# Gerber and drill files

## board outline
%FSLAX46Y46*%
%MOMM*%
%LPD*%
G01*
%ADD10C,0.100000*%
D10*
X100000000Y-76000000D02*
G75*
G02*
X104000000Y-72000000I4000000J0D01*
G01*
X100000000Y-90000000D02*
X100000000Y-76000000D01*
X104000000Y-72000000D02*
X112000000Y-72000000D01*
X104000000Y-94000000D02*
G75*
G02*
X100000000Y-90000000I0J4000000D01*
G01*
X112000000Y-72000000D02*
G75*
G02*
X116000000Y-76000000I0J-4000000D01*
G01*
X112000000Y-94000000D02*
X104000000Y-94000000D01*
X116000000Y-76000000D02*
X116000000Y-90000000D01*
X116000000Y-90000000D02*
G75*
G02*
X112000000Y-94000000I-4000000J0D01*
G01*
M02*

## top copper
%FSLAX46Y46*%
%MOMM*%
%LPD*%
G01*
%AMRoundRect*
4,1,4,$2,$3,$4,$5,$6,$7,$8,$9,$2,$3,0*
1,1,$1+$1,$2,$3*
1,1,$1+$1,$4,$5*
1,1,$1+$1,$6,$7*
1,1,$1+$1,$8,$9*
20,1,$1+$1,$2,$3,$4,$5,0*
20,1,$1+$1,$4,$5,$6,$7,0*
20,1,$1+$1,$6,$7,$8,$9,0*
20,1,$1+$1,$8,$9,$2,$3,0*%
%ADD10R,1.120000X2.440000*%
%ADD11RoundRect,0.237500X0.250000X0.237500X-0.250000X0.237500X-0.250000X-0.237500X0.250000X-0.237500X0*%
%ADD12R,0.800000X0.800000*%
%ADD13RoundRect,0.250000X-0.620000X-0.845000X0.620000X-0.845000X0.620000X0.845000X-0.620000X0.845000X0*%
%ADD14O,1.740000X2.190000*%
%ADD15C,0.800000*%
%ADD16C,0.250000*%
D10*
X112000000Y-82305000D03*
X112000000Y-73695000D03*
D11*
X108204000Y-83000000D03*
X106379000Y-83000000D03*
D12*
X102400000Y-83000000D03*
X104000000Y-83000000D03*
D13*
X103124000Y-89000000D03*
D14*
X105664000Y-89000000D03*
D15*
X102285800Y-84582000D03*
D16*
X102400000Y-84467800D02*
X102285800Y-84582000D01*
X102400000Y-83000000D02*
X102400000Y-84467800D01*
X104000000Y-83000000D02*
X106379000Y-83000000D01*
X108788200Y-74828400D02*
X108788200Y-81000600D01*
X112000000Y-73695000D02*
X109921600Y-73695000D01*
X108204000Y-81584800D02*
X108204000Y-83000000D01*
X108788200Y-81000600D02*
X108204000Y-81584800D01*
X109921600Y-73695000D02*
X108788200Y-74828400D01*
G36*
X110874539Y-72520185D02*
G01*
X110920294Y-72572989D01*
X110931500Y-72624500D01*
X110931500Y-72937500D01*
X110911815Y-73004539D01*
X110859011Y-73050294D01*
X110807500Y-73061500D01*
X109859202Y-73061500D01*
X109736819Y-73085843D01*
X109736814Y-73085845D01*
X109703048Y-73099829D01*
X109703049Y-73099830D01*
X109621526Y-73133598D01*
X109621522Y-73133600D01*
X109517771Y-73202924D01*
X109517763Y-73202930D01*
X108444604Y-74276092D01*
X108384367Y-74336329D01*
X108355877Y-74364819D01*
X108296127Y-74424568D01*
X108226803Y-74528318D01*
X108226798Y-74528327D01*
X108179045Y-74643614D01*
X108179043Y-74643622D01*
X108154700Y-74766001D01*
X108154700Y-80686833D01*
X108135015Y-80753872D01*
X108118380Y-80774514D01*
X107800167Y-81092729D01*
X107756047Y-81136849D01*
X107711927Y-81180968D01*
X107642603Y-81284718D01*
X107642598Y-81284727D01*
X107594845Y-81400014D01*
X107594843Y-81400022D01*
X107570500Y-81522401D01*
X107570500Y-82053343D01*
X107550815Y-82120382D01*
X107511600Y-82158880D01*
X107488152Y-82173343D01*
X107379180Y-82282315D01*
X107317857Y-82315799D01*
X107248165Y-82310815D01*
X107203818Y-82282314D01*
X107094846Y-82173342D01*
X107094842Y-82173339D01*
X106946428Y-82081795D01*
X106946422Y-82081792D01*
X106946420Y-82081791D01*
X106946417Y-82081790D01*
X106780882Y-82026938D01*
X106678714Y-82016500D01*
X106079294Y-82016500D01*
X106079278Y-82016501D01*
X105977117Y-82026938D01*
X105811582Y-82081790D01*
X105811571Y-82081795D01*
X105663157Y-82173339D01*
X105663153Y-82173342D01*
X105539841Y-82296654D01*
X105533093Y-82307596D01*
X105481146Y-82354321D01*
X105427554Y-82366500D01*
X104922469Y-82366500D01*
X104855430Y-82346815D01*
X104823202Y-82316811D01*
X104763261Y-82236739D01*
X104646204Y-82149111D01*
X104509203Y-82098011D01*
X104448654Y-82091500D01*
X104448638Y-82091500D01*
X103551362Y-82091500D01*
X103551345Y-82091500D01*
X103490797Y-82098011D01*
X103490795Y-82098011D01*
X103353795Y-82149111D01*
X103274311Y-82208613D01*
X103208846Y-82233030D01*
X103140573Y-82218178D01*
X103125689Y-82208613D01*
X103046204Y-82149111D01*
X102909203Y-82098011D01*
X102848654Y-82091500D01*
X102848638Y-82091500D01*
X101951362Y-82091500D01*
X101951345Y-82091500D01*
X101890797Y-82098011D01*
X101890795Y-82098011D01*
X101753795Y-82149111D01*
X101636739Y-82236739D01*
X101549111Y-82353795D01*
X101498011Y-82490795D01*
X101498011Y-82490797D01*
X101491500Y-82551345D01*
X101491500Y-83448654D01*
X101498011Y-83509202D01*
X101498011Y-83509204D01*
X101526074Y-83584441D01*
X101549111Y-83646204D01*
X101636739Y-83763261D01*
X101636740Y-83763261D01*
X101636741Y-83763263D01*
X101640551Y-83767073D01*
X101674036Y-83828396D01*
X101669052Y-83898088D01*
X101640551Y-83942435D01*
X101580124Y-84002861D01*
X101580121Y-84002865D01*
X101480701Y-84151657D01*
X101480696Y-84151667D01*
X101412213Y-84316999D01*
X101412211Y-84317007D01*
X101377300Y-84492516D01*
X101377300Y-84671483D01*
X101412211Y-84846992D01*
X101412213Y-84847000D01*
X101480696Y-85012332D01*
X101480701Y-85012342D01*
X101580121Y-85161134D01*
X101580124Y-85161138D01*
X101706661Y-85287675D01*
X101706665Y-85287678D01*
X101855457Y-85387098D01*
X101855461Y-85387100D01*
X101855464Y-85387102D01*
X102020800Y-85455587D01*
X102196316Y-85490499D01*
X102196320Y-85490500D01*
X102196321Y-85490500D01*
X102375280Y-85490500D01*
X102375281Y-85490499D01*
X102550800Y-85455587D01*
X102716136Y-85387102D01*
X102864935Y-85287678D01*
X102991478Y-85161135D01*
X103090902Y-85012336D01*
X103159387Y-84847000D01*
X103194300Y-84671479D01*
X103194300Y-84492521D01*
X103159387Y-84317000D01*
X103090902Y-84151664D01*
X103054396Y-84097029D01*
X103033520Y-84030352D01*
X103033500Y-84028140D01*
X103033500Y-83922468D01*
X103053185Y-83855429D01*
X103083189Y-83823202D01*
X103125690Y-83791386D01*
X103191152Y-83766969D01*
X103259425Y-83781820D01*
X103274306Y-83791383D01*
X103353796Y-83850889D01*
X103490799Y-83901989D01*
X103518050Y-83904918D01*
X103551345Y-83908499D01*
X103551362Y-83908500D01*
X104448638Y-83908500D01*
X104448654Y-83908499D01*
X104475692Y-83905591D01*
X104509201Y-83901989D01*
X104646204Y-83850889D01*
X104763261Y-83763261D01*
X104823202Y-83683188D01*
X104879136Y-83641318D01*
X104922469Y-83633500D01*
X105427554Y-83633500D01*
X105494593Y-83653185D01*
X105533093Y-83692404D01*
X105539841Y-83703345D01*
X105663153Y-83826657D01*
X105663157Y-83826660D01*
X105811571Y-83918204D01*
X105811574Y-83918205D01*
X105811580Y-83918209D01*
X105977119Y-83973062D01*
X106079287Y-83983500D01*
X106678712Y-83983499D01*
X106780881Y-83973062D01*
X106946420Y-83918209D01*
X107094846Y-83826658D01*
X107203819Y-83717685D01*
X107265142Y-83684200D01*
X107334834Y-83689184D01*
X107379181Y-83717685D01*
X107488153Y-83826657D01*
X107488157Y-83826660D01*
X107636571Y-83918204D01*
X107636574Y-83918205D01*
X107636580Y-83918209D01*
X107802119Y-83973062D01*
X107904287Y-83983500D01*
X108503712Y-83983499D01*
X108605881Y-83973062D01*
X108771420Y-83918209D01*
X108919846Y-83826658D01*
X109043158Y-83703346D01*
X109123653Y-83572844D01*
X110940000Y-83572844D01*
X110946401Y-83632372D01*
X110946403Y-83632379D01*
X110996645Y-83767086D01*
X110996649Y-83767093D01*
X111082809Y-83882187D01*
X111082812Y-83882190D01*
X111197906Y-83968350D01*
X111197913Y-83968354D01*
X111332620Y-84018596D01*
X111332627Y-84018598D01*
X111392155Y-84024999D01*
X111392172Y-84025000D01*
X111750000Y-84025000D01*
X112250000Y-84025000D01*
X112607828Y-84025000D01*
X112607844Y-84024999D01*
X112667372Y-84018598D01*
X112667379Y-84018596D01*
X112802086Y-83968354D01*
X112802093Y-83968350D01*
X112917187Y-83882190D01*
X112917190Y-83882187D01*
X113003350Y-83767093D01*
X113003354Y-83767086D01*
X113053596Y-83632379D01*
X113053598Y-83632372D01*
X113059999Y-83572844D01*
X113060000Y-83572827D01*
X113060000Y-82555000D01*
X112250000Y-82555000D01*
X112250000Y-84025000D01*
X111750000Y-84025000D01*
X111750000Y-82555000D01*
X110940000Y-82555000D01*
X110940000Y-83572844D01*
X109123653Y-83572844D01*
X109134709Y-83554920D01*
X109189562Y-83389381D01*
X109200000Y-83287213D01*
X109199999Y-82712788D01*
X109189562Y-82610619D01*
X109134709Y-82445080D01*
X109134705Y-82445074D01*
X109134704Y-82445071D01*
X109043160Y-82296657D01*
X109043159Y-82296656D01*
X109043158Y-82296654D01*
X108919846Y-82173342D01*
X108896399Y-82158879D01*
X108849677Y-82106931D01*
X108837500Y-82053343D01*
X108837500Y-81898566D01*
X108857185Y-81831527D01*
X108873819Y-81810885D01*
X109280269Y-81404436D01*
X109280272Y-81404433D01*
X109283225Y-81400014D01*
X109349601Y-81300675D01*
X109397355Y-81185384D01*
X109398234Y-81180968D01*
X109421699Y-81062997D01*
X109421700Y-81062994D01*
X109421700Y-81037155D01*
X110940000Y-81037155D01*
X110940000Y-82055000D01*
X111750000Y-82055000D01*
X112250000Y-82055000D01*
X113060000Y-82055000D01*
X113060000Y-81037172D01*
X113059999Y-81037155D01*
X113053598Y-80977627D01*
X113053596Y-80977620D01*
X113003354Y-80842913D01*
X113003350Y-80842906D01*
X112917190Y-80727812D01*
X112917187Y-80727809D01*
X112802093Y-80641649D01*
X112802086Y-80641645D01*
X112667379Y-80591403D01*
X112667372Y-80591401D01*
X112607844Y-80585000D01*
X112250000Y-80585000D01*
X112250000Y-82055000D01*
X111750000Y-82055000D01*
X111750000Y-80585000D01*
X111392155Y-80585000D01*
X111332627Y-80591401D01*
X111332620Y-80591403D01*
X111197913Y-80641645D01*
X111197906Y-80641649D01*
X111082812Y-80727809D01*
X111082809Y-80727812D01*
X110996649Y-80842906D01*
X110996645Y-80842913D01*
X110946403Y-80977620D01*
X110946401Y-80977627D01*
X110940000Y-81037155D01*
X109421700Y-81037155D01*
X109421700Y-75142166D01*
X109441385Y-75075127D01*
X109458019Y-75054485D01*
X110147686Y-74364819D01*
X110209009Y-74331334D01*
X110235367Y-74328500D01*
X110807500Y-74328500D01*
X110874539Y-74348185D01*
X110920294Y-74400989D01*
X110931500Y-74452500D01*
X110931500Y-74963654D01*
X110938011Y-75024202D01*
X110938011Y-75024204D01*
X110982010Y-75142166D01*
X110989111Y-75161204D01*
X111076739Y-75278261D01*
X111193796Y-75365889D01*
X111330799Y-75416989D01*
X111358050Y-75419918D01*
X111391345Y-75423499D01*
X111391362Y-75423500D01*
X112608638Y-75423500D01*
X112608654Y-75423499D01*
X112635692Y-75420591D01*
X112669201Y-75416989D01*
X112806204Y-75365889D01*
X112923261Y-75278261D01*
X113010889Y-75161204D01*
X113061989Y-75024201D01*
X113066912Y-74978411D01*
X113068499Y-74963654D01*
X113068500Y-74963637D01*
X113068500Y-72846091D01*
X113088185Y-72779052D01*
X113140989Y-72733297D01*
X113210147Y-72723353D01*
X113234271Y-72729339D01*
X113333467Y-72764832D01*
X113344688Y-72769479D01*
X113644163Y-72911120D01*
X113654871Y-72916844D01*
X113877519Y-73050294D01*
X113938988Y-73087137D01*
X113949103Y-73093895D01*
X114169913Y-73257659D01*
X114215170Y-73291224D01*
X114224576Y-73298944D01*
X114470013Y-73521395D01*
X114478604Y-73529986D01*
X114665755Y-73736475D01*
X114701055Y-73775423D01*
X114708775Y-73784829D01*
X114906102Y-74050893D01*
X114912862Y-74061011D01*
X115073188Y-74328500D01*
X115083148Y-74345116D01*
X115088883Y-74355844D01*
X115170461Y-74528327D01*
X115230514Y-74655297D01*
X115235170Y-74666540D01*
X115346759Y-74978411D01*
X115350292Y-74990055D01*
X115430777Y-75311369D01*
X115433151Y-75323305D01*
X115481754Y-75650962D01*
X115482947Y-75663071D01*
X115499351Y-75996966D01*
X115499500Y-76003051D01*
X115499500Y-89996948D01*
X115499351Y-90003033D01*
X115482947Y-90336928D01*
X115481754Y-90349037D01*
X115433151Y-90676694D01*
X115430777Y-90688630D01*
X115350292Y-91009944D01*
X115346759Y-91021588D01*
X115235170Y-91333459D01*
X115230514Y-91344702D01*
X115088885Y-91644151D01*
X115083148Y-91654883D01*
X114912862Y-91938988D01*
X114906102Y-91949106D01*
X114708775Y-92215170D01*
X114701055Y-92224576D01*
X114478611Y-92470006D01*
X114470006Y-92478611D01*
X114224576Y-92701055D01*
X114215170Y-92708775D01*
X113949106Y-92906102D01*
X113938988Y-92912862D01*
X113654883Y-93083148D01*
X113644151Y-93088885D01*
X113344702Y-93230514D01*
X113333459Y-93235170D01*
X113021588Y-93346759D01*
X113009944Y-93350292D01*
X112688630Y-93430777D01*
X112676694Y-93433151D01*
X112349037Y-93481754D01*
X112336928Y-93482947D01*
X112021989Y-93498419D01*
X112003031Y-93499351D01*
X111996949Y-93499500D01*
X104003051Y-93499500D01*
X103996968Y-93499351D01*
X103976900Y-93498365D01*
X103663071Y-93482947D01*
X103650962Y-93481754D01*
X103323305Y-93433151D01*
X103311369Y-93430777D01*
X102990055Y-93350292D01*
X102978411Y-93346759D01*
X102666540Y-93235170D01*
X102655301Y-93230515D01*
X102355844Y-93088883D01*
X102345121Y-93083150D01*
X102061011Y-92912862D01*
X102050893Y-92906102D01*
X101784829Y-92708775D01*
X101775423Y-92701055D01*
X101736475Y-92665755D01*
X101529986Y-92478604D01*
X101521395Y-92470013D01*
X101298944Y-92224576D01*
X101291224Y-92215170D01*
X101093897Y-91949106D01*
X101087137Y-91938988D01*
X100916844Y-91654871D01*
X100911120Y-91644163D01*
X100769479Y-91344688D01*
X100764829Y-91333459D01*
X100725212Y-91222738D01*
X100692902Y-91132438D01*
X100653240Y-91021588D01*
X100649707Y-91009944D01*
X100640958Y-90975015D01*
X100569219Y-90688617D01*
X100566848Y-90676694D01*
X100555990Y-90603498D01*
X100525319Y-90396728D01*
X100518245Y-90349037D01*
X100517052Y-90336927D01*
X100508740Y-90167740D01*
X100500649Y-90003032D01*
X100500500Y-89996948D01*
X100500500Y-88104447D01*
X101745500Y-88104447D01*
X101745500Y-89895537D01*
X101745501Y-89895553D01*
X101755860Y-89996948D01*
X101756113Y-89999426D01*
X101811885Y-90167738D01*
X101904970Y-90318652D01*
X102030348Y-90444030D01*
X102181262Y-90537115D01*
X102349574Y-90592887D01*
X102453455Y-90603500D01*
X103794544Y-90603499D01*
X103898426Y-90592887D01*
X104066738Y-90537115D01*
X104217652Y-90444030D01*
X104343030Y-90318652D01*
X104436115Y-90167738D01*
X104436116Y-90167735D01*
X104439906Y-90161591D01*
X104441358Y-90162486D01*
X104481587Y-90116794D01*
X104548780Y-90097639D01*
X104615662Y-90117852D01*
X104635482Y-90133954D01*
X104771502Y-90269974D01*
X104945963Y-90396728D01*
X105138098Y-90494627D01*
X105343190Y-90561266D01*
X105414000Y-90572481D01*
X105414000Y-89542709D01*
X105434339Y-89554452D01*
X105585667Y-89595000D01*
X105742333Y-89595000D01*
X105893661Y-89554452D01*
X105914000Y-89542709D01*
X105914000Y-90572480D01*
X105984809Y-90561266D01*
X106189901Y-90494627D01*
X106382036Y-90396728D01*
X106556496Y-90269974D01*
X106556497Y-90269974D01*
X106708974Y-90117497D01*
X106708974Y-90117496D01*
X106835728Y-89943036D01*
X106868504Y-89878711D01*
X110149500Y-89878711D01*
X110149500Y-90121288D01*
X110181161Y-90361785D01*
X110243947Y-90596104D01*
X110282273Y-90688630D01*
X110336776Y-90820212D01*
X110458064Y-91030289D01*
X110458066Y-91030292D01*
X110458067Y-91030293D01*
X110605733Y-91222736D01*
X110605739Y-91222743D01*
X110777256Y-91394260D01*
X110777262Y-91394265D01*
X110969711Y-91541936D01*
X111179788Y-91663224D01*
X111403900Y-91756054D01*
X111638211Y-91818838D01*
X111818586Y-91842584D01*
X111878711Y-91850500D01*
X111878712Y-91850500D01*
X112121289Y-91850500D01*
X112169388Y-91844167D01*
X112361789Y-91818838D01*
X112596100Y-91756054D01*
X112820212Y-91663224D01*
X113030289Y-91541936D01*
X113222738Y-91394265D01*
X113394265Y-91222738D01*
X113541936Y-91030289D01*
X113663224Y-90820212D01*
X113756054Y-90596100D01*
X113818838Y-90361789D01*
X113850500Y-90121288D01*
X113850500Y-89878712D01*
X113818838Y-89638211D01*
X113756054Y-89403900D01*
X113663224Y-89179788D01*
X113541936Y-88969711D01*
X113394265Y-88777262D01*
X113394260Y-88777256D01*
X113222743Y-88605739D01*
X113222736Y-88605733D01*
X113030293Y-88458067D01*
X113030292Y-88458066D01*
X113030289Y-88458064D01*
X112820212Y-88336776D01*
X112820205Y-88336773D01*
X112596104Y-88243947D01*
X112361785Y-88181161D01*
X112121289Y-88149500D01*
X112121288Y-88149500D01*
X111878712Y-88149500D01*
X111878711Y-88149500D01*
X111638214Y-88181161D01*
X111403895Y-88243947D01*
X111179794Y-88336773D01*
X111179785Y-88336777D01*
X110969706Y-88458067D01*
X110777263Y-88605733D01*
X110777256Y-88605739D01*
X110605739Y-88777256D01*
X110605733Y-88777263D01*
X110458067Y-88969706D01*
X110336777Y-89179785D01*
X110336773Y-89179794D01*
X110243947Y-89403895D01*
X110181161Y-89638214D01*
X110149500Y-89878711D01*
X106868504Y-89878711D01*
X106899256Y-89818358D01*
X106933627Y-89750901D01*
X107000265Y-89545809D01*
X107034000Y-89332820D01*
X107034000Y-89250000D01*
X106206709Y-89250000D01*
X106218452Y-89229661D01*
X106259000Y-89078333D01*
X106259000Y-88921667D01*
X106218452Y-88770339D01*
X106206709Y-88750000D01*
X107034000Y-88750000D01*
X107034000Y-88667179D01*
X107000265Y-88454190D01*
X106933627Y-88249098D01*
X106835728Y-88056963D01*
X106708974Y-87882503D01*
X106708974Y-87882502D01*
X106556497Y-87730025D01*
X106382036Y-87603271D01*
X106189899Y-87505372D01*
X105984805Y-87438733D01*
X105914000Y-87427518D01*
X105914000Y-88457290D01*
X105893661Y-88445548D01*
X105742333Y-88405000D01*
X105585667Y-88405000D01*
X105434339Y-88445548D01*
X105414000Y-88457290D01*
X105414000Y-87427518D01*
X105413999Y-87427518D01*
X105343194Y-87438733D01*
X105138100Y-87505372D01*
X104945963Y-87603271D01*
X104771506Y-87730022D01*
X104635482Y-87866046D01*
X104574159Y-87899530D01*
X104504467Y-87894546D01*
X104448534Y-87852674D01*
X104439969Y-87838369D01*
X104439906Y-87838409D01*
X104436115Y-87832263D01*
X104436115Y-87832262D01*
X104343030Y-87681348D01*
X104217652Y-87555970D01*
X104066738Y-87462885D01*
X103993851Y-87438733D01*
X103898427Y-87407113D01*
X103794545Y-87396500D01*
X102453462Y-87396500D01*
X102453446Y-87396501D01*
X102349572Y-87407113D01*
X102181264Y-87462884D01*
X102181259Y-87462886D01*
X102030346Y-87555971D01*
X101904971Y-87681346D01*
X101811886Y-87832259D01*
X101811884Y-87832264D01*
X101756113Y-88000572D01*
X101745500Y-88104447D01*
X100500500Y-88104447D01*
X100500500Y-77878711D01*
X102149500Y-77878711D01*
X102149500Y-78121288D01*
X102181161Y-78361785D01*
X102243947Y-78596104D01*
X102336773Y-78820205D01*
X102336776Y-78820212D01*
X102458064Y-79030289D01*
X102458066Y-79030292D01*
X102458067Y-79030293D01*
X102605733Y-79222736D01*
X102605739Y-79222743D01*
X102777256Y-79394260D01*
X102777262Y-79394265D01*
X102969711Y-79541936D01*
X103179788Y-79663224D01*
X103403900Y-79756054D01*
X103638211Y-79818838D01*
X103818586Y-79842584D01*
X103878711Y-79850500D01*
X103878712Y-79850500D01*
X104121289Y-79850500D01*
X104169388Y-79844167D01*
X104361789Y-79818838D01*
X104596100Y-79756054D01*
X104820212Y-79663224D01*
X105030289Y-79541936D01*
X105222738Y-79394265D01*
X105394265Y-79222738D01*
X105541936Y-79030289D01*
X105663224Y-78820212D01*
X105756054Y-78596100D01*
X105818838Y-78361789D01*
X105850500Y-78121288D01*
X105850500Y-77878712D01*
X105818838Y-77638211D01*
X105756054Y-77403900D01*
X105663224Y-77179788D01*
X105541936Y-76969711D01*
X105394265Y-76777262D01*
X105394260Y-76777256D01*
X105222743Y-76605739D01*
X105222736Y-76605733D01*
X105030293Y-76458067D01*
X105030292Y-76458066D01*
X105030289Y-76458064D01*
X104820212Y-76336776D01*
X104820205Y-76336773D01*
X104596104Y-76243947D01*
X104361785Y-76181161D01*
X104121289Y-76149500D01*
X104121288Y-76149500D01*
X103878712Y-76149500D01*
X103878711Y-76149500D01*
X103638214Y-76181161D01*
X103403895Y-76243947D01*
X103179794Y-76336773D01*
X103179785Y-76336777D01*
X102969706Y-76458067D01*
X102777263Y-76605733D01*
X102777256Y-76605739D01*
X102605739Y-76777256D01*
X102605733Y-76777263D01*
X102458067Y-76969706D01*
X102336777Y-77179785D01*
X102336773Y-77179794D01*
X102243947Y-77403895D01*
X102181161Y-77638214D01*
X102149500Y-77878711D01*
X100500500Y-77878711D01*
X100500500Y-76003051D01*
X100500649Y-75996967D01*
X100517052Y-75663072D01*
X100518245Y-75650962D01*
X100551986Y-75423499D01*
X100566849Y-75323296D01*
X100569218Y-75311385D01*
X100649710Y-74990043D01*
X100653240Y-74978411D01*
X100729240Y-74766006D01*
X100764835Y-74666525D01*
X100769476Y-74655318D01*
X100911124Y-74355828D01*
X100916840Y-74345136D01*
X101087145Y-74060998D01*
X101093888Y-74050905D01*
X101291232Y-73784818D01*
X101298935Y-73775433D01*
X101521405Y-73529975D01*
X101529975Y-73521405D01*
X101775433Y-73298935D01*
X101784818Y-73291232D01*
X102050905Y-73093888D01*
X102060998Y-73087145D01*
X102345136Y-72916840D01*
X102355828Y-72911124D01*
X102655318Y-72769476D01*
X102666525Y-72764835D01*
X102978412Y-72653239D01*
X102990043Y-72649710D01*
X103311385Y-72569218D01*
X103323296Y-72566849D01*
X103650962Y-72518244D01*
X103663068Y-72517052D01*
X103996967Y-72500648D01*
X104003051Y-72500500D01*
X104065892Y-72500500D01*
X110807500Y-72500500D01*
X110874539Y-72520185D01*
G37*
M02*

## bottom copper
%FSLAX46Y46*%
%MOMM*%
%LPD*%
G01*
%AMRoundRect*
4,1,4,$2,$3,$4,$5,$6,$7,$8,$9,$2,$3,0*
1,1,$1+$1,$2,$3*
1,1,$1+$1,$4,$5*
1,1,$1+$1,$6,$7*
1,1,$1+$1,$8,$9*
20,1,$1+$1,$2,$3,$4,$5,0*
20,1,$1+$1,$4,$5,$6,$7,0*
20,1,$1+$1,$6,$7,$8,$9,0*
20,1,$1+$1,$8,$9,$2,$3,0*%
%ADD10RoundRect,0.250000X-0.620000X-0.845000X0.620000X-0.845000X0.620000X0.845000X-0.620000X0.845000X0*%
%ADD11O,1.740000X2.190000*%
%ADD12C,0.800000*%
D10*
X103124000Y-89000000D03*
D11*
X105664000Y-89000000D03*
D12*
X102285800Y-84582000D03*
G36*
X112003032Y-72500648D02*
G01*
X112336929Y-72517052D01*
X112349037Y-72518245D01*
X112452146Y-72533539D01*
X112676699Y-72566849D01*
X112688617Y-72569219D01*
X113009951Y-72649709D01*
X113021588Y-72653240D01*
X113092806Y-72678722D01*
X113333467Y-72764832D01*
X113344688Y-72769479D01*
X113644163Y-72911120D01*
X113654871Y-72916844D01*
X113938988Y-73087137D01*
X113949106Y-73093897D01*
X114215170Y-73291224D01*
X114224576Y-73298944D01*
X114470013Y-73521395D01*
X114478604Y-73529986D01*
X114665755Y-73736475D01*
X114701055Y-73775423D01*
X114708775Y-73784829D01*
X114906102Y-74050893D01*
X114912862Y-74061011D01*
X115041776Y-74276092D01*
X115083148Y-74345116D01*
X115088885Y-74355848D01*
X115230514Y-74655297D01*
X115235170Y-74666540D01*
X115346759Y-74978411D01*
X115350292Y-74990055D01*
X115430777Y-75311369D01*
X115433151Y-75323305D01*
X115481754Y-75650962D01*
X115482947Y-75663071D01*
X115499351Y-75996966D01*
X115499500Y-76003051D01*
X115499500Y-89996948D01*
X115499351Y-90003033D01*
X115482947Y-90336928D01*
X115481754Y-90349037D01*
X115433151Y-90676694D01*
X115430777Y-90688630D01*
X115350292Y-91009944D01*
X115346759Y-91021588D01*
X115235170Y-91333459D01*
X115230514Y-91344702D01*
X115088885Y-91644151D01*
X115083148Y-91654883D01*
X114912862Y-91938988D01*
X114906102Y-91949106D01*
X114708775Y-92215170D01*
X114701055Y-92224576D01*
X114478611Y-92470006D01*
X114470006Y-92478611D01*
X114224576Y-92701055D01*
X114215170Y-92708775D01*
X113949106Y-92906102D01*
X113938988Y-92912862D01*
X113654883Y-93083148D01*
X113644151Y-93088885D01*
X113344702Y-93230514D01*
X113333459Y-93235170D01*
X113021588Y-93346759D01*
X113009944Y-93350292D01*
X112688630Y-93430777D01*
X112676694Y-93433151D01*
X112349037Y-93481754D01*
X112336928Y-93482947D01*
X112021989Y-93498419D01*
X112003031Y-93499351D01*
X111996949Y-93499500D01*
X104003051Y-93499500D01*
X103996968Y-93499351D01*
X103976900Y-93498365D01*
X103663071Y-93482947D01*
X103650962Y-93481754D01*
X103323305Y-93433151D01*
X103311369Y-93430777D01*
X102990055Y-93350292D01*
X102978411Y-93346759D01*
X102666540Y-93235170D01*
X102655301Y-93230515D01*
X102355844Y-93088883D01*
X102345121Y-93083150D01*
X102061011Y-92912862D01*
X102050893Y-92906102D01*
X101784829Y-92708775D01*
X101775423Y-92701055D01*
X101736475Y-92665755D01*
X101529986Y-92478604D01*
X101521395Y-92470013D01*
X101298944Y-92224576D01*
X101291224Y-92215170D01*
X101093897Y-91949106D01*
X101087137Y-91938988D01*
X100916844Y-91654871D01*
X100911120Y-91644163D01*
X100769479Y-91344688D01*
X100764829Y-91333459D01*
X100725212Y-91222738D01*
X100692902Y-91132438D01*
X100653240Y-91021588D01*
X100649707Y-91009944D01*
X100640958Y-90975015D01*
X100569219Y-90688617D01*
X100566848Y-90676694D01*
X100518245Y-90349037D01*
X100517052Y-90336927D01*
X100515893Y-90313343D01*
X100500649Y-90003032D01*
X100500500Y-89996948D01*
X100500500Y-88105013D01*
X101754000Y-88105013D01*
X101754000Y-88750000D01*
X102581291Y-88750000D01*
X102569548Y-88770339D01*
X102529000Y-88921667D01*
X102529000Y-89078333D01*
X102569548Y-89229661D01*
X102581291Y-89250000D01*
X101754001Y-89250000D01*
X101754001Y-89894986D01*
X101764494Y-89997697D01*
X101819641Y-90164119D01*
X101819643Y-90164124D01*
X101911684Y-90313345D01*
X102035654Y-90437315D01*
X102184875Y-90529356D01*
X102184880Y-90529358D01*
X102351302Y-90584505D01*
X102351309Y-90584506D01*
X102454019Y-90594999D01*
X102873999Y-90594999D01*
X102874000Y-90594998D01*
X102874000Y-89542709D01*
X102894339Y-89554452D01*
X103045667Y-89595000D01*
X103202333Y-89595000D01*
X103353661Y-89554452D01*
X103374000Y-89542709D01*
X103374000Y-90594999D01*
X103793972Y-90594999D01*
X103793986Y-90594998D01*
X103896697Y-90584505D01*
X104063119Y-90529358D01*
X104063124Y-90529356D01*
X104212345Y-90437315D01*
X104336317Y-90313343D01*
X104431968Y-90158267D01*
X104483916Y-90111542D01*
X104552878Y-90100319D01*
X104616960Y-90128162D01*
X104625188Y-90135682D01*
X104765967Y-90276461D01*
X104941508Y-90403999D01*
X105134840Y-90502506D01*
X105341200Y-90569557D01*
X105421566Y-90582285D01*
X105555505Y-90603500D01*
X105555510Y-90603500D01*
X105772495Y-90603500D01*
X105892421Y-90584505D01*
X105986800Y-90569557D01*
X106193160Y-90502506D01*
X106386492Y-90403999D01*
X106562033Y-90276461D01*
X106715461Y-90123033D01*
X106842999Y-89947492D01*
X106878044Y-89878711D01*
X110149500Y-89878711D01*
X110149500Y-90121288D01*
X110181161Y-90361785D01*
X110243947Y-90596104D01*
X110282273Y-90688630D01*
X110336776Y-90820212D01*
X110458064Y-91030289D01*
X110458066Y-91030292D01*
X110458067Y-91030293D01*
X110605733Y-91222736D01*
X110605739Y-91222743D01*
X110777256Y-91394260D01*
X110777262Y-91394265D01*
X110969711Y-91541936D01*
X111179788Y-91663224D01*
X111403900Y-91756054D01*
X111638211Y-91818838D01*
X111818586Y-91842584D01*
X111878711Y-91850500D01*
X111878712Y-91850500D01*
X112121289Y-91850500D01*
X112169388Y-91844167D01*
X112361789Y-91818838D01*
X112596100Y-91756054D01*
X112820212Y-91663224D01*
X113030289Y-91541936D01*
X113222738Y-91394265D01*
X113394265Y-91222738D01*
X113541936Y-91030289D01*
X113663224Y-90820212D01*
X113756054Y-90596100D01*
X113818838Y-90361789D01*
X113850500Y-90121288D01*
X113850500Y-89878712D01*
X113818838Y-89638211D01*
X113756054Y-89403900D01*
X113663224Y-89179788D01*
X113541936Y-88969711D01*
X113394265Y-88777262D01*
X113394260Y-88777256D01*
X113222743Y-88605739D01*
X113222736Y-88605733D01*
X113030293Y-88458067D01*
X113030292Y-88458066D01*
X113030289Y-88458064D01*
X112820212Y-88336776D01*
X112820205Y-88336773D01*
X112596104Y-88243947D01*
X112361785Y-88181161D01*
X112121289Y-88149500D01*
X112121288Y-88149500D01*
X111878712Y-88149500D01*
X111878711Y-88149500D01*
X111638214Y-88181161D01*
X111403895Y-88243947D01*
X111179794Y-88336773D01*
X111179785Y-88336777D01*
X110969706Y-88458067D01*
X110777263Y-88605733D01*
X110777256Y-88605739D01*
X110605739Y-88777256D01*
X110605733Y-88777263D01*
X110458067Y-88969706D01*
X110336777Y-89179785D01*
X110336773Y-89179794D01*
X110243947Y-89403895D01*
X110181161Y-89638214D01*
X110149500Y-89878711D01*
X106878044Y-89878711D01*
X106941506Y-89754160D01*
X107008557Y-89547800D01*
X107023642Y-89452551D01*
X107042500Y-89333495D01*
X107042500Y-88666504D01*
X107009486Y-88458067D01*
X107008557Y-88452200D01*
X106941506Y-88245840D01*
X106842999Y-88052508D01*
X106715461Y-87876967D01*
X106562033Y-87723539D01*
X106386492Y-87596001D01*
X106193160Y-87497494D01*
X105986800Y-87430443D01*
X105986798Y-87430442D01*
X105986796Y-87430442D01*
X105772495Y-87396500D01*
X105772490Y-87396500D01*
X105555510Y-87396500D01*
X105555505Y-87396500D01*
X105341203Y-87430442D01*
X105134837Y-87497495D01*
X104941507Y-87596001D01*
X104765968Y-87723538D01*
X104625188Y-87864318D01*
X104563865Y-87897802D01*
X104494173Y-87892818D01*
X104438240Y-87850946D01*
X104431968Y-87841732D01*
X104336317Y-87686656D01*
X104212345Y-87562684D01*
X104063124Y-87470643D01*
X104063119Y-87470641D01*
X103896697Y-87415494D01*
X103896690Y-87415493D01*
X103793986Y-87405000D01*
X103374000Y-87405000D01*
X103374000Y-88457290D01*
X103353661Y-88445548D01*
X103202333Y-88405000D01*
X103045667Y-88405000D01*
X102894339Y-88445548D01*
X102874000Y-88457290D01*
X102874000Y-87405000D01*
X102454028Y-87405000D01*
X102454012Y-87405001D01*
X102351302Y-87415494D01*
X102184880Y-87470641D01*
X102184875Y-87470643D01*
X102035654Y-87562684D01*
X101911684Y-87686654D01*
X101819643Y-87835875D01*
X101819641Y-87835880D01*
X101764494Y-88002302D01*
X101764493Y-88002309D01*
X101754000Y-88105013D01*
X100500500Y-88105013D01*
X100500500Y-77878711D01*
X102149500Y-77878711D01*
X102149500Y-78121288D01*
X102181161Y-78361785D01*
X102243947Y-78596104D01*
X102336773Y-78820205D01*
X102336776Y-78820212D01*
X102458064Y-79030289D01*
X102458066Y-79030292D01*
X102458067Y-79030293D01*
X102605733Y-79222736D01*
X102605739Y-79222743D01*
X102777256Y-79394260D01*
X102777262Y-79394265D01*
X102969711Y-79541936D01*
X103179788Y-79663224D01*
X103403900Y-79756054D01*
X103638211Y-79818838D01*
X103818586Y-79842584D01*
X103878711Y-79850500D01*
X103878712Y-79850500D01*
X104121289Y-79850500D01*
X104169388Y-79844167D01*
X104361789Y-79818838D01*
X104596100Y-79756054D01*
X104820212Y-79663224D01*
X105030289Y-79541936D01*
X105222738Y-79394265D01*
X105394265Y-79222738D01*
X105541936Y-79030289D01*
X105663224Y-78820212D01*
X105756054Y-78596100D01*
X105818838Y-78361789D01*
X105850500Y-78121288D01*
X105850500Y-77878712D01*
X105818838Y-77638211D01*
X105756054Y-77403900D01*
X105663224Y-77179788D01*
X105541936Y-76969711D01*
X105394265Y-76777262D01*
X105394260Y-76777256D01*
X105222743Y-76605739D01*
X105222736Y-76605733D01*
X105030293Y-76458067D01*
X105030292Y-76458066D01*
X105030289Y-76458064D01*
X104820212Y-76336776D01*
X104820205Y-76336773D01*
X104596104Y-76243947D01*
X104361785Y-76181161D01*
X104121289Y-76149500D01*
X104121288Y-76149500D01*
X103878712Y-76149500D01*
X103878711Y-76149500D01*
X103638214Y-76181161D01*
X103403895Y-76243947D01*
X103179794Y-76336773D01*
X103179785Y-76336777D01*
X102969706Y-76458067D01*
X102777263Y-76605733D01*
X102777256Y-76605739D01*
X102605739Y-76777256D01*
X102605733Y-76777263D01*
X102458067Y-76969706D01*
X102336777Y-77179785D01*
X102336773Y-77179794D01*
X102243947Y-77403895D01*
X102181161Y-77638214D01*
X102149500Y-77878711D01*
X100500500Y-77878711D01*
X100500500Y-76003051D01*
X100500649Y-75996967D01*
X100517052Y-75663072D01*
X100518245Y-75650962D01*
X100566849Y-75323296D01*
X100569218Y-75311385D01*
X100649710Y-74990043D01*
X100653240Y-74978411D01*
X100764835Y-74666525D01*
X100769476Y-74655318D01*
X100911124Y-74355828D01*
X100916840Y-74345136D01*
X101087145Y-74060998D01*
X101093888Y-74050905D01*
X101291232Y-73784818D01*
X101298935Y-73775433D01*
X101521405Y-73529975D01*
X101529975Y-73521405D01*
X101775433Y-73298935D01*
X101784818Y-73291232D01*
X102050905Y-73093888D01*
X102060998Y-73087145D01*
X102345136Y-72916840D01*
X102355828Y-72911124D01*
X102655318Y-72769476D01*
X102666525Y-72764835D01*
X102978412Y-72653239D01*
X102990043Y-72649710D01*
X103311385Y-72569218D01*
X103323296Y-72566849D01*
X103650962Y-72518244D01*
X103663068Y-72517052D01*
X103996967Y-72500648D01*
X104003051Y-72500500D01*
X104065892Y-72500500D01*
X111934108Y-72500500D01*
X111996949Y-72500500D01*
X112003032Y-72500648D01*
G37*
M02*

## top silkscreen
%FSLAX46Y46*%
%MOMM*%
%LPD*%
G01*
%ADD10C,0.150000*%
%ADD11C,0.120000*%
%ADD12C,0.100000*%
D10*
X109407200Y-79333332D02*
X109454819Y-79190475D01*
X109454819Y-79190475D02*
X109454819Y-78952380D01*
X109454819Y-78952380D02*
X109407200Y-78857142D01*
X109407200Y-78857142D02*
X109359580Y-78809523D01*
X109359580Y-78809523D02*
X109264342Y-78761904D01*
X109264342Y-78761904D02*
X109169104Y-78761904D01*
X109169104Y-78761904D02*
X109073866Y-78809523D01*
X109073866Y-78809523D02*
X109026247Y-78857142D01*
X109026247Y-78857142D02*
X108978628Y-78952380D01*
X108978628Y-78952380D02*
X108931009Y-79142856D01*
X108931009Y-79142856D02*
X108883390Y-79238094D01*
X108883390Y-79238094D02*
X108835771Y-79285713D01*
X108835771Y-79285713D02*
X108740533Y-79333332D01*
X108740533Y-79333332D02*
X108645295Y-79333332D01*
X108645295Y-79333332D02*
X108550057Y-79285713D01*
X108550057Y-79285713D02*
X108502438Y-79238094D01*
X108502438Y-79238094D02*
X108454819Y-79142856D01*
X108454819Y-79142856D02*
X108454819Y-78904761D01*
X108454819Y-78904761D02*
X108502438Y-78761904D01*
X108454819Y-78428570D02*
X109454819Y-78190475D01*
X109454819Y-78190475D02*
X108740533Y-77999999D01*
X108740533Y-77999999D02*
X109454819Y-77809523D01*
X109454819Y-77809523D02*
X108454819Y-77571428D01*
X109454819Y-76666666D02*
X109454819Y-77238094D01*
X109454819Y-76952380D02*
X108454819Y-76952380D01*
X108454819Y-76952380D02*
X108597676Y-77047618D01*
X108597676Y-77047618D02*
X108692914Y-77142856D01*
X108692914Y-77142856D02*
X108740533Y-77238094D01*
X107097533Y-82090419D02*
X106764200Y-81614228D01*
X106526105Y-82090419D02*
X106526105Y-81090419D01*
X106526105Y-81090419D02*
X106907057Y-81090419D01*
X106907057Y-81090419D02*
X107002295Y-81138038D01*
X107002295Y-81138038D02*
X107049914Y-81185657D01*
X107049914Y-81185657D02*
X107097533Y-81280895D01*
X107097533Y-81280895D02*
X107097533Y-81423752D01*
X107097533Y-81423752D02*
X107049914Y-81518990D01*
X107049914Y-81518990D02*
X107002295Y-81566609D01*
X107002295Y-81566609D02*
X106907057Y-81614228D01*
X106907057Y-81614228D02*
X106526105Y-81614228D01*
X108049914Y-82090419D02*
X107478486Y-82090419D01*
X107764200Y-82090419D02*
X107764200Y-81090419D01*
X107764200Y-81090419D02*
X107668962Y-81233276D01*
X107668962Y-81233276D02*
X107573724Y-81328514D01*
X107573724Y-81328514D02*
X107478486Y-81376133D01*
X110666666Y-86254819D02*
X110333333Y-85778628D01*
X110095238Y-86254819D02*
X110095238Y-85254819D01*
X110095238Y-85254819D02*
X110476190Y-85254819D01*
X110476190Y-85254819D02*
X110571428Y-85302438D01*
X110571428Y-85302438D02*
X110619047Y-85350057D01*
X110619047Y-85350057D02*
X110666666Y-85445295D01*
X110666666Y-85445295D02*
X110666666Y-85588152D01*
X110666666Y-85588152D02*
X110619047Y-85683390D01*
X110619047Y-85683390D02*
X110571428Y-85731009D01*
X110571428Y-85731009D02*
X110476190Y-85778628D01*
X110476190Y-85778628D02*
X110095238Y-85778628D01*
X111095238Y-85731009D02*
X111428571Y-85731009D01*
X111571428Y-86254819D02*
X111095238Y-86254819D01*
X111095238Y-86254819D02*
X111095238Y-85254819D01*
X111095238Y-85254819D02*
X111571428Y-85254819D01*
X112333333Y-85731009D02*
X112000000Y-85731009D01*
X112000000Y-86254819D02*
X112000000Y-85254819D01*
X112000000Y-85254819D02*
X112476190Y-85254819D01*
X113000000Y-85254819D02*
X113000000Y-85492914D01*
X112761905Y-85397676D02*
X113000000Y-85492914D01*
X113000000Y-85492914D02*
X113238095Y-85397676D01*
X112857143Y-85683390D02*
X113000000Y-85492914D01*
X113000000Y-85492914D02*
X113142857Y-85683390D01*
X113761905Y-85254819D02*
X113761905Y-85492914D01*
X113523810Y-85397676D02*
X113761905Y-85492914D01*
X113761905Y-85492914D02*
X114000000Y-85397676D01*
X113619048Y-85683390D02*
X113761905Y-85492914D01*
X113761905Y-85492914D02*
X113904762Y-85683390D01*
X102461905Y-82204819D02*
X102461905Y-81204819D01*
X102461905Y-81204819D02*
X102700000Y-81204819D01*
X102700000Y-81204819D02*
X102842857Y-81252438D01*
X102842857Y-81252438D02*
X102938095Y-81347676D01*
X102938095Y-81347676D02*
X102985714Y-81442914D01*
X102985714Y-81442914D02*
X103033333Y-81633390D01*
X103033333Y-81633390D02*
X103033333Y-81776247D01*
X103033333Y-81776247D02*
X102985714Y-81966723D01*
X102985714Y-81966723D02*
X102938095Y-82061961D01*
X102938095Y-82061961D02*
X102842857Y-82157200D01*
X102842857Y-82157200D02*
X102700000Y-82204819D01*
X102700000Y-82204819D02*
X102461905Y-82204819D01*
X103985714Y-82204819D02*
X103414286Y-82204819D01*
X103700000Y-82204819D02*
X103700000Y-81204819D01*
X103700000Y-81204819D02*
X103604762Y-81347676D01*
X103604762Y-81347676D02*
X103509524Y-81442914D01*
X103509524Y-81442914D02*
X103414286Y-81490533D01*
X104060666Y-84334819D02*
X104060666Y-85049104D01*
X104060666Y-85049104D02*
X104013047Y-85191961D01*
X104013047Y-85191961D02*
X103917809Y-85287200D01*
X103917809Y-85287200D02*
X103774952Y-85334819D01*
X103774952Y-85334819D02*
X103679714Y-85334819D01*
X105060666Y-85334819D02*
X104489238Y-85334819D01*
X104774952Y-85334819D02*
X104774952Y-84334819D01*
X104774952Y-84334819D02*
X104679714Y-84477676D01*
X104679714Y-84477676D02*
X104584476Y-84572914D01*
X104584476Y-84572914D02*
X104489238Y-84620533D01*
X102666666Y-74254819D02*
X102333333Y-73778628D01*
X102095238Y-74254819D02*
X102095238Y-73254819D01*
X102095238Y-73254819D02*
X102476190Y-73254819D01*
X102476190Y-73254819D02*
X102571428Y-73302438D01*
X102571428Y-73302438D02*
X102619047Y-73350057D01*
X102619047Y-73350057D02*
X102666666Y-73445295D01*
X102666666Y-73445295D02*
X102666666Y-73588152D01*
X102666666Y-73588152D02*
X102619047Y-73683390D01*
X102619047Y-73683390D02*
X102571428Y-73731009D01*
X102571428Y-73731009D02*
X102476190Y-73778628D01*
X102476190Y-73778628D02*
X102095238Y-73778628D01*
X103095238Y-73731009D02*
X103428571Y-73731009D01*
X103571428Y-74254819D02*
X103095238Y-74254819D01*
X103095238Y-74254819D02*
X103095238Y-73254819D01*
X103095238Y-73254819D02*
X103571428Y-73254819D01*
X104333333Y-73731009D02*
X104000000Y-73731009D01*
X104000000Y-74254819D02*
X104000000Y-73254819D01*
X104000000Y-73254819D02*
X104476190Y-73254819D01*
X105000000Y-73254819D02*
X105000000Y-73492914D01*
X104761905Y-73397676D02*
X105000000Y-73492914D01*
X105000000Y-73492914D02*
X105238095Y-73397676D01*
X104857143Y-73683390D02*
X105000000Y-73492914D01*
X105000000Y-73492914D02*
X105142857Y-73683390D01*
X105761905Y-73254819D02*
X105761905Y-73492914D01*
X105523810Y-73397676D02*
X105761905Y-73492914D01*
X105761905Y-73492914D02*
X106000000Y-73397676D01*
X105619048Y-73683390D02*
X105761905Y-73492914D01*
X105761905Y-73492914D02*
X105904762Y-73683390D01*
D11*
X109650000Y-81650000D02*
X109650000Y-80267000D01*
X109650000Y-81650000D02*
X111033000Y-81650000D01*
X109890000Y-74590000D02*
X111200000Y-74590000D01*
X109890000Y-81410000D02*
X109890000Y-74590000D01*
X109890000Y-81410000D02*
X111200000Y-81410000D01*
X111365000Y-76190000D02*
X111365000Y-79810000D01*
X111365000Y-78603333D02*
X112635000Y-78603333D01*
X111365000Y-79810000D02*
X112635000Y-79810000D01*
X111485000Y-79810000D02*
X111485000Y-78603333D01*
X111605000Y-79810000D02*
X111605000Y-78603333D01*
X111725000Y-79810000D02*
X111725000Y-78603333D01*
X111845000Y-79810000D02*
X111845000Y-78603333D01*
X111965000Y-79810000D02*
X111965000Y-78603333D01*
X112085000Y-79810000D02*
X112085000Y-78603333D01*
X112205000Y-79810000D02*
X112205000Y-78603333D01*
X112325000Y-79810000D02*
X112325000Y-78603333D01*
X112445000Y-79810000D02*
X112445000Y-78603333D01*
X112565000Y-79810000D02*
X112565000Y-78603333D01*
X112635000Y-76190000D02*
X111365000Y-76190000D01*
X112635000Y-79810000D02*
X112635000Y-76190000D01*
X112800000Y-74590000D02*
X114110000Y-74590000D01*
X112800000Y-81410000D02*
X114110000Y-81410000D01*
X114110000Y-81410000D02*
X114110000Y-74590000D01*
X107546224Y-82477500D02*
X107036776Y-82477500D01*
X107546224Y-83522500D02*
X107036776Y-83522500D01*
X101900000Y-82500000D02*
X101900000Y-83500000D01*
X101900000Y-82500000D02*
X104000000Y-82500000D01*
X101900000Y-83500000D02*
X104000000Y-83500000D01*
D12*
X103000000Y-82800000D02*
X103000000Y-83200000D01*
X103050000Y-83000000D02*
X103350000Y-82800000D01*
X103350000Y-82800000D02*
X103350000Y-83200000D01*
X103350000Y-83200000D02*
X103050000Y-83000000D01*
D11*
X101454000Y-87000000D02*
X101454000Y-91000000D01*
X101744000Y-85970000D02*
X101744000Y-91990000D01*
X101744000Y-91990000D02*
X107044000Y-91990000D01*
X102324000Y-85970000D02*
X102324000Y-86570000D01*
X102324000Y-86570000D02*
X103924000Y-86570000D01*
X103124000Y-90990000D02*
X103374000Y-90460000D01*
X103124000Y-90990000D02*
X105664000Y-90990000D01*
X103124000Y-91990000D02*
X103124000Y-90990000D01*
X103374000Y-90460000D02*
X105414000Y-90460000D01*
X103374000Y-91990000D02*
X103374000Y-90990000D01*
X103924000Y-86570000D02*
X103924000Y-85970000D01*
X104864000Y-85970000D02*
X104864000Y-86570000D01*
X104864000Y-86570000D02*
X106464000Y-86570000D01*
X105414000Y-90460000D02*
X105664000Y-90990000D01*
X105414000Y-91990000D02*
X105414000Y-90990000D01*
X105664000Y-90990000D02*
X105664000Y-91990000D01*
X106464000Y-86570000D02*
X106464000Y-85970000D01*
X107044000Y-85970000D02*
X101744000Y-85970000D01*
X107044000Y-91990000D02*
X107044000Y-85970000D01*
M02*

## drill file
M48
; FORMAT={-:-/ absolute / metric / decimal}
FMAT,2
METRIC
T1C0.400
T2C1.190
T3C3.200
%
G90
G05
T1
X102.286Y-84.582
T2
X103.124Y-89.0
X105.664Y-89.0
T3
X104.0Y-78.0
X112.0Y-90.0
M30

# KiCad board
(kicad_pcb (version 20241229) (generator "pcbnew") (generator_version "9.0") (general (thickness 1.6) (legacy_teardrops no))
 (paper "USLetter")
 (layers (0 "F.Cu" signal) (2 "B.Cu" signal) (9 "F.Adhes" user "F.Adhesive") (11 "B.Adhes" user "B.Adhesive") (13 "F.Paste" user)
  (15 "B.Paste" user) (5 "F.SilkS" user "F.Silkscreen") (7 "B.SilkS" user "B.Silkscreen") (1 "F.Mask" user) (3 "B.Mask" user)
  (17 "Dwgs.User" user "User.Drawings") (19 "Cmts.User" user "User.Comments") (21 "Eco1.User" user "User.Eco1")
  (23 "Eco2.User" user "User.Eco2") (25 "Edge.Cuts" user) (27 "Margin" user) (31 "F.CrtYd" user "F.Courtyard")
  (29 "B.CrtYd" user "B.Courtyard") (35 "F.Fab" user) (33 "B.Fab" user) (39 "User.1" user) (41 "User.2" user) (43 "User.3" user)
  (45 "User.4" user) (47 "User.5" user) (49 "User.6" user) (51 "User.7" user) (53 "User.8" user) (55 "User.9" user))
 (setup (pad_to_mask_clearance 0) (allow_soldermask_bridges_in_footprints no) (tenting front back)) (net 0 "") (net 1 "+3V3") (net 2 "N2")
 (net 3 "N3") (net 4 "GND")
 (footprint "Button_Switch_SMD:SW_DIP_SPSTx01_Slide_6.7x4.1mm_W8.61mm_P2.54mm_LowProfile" (layer "F.Cu") (at 112 78 90)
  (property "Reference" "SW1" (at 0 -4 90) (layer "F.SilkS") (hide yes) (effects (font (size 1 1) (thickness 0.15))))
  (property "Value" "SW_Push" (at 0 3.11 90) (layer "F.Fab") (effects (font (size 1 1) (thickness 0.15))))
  (fp_line (start -3.65 -2.35) (end -2.267 -2.35) (stroke (width 0.12) (type solid)) (layer "F.SilkS"))
  (fp_line (start -3.65 -2.35) (end -3.65 -0.967) (stroke (width 0.12) (type solid)) (layer "F.SilkS"))
  (fp_line (start 3.41 -2.11) (end 3.41 -0.8) (stroke (width 0.12) (type solid)) (layer "F.SilkS"))
  (fp_line (start -3.41 -2.11) (end 3.41 -2.11) (stroke (width 0.12) (type solid)) (layer "F.SilkS"))
  (fp_line (start -3.41 -2.11) (end -3.41 -0.8) (stroke (width 0.12) (type solid)) (layer "F.SilkS"))
  (fp_line (start 1.81 -0.635) (end -1.81 -0.635) (stroke (width 0.12) (type solid)) (layer "F.SilkS"))
  (fp_line (start -0.603333 -0.635) (end -0.603333 0.635) (stroke (width 0.12) (type solid)) (layer "F.SilkS"))
  (fp_line (start -1.81 -0.635) (end -1.81 0.635) (stroke (width 0.12) (type solid)) (layer "F.SilkS"))
  (fp_line (start -1.81 -0.515) (end -0.603333 -0.515) (stroke (width 0.12) (type solid)) (layer "F.SilkS"))
  (fp_line (start -1.81 -0.395) (end -0.603333 -0.395) (stroke (width 0.12) (type solid)) (layer "F.SilkS"))
  (fp_line (start -1.81 -0.275) (end -0.603333 -0.275) (stroke (width 0.12) (type solid)) (layer "F.SilkS"))
  (fp_line (start -1.81 -0.155) (end -0.603333 -0.155) (stroke (width 0.12) (type solid)) (layer "F.SilkS"))
  (fp_line (start -1.81 -0.035) (end -0.603333 -0.035) (stroke (width 0.12) (type solid)) (layer "F.SilkS"))
  (fp_line (start -1.81 0.085) (end -0.603333 0.085) (stroke (width 0.12) (type solid)) (layer "F.SilkS"))
  (fp_line (start -1.81 0.205) (end -0.603333 0.205) (stroke (width 0.12) (type solid)) (layer "F.SilkS"))
  (fp_line (start -1.81 0.325) (end -0.603333 0.325) (stroke (width 0.12) (type solid)) (layer "F.SilkS"))
  (fp_line (start -1.81 0.445) (end -0.603333 0.445) (stroke (width 0.12) (type solid)) (layer "F.SilkS"))
  (fp_line (start -1.81 0.565) (end -0.603333 0.565) (stroke (width 0.12) (type solid)) (layer "F.SilkS"))
  (fp_line (start 1.81 0.635) (end 1.81 -0.635) (stroke (width 0.12) (type solid)) (layer "F.SilkS"))
  (fp_line (start -1.81 0.635) (end 1.81 0.635) (stroke (width 0.12) (type solid)) (layer "F.SilkS"))
  (fp_line (start 3.41 0.8) (end 3.41 2.11) (stroke (width 0.12) (type solid)) (layer "F.SilkS"))
  (fp_line (start -3.41 0.8) (end -3.41 2.11) (stroke (width 0.12) (type solid)) (layer "F.SilkS"))
  (fp_line (start -3.41 2.11) (end 3.41 2.11) (stroke (width 0.12) (type solid)) (layer "F.SilkS"))
  (pad "1" smd rect (at -4.305 0 90) (size 2.44 1.12) (layers "F.Cu" "F.Mask" "F.Paste") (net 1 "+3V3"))
  (pad "2" smd rect (at 4.305 0 90) (size 2.44 1.12) (layers "F.Cu" "F.Mask" "F.Paste") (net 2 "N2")))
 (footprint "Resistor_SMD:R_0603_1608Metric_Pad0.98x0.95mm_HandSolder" (layer "F.Cu") (at 107.2915 83 180)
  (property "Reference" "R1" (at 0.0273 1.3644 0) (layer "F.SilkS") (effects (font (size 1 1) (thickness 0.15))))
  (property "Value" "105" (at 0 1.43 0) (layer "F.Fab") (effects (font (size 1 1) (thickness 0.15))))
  (fp_line (start -0.254724 0.5225) (end 0.254724 0.5225) (stroke (width 0.12) (type solid)) (layer "F.SilkS"))
  (fp_line (start -0.254724 -0.5225) (end 0.254724 -0.5225) (stroke (width 0.12) (type solid)) (layer "F.SilkS"))
  (pad "1" smd roundrect (at -0.9125 0 180) (size 0.975 0.95) (layers "F.Cu" "F.Mask" "F.Paste") (roundrect_rratio 0.25) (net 2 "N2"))
  (pad "2" smd roundrect (at 0.9125 0 180) (size 0.975 0.95) (layers "F.Cu" "F.Mask" "F.Paste") (roundrect_rratio 0.25) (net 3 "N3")))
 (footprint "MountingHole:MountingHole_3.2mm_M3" (layer "F.Cu") (at 112 90)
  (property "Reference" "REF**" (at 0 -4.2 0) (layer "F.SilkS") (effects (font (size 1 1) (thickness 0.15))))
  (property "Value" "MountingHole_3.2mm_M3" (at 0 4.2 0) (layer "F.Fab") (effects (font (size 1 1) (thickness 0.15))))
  (pad "" np_thru_hole circle (at 0 0) (size 3.2 3.2) (drill 3.2) (layers "*.Cu" "*.Mask")))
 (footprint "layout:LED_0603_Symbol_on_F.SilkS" (layer "F.Cu") (at 103.2 83)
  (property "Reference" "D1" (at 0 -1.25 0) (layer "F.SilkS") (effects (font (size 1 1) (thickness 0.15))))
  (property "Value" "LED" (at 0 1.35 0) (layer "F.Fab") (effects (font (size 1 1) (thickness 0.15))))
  (fp_line (start -1.3 -0.5) (end -1.3 0.5) (stroke (width 0.12) (type solid)) (layer "F.SilkS"))
  (fp_line (start -1.3 -0.5) (end 0.8 -0.5) (stroke (width 0.12) (type solid)) (layer "F.SilkS"))
  (fp_line (start -1.3 0.5) (end 0.8 0.5) (stroke (width 0.12) (type solid)) (layer "F.SilkS"))
  (fp_line (start -0.2 -0.2) (end -0.2 0.2) (stroke (width 0.1) (type solid)) (layer "F.SilkS"))
  (fp_line (start -0.15 0) (end 0.15 -0.2) (stroke (width 0.1) (type solid)) (layer "F.SilkS"))
  (fp_line (start 0.15 -0.2) (end 0.15 0.2) (stroke (width 0.1) (type solid)) (layer "F.SilkS"))
  (fp_line (start 0.15 0.2) (end -0.15 0) (stroke (width 0.1) (type solid)) (layer "F.SilkS"))
  (pad "1" smd rect (at -0.8 0 180) (size 0.8 0.8) (layers "F.Cu" "F.Mask" "F.Paste") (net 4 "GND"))
  (pad "2" smd rect (at 0.8 0 180) (size 0.8 0.8) (layers "F.Cu" "F.Mask" "F.Paste") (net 3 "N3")))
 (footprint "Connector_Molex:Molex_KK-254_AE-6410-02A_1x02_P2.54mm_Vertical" (layer "F.Cu") (at 103.124 89)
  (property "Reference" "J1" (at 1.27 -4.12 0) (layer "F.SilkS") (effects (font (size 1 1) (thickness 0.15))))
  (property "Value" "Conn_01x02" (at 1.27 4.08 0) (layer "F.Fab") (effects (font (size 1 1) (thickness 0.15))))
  (fp_line (start -1.67 -2) (end -1.67 2) (stroke (width 0.12) (type solid)) (layer "F.SilkS"))
  (fp_line (start -1.38 -3.03) (end -1.38 2.99) (stroke (width 0.12) (type solid)) (layer "F.SilkS"))
  (fp_line (start -1.38 2.99) (end 3.92 2.99) (stroke (width 0.12) (type solid)) (layer "F.SilkS"))
  (fp_line (start -0.8 -3.03) (end -0.8 -2.43) (stroke (width 0.12) (type solid)) (layer "F.SilkS"))
  (fp_line (start -0.8 -2.43) (end 0.8 -2.43) (stroke (width 0.12) (type solid)) (layer "F.SilkS"))
  (fp_line (start 0 1.99) (end 0.25 1.46) (stroke (width 0.12) (type solid)) (layer "F.SilkS"))
  (fp_line (start 0 1.99) (end 2.54 1.99) (stroke (width 0.12) (type solid)) (layer "F.SilkS"))
  (fp_line (start 0 2.99) (end 0 1.99) (stroke (width 0.12) (type solid)) (layer "F.SilkS"))
  (fp_line (start 0.25 1.46) (end 2.29 1.46) (stroke (width 0.12) (type solid)) (layer "F.SilkS"))
  (fp_line (start 0.25 2.99) (end 0.25 1.99) (stroke (width 0.12) (type solid)) (layer "F.SilkS"))
  (fp_line (start 0.8 -2.43) (end 0.8 -3.03) (stroke (width 0.12) (type solid)) (layer "F.SilkS"))
  (fp_line (start 1.74 -3.03) (end 1.74 -2.43) (stroke (width 0.12) (type solid)) (layer "F.SilkS"))
  (fp_line (start 1.74 -2.43) (end 3.34 -2.43) (stroke (width 0.12) (type solid)) (layer "F.SilkS"))
  (fp_line (start 2.29 1.46) (end 2.54 1.99) (stroke (width 0.12) (type solid)) (layer "F.SilkS"))
  (fp_line (start 2.29 2.99) (end 2.29 1.99) (stroke (width 0.12) (type solid)) (layer "F.SilkS"))
  (fp_line (start 2.54 1.99) (end 2.54 2.99) (stroke (width 0.12) (type solid)) (layer "F.SilkS"))
  (fp_line (start 3.34 -2.43) (end 3.34 -3.03) (stroke (width 0.12) (type solid)) (layer "F.SilkS"))
  (fp_line (start 3.92 -3.03) (end -1.38 -3.03) (stroke (width 0.12) (type solid)) (layer "F.SilkS"))
  (fp_line (start 3.92 2.99) (end 3.92 -3.03) (stroke (width 0.12) (type solid)) (layer "F.SilkS"))
  (pad "1" thru_hole roundrect (at 0 0) (size 1.74 2.19) (drill 1.19) (layers "*.Cu" "*.Mask") (remove_unused_layers no)
   (roundrect_rratio 0.143678) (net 4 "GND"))
  (pad "2" thru_hole oval (at 2.54 0) (size 1.74 2.19) (drill 1.19) (layers "*.Cu" "*.Mask") (remove_unused_layers no) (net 1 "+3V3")))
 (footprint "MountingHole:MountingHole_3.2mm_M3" (layer "F.Cu") (at 104 78)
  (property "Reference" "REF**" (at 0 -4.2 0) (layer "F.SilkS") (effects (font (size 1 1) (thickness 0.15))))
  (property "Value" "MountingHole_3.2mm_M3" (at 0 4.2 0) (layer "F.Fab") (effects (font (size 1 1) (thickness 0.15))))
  (pad "" np_thru_hole circle (at 0 0) (size 3.2 3.2) (drill 3.2) (layers "*.Cu" "*.Mask")))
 (gr_arc (start 100 76) (mid 101.171573 73.171573) (end 104 72) (stroke (width 0.1) (type default)) (layer "Edge.Cuts"))
 (gr_line (start 100 90) (end 100 76) (stroke (width 0.1) (type default)) (layer "Edge.Cuts"))
 (gr_line (start 104 72) (end 112 72) (stroke (width 0.1) (type default)) (layer "Edge.Cuts"))
 (gr_arc (start 104 94) (mid 101.171573 92.828427) (end 100 90) (stroke (width 0.1) (type default)) (layer "Edge.Cuts"))
 (gr_arc (start 112 72) (mid 114.828427 73.171573) (end 116 76) (stroke (width 0.1) (type default)) (layer "Edge.Cuts"))
 (gr_line (start 112 94) (end 104 94) (stroke (width 0.1) (type default)) (layer "Edge.Cuts"))
 (gr_line (start 116 76) (end 116 90) (stroke (width 0.1) (type default)) (layer "Edge.Cuts"))
 (gr_arc (start 116 90) (mid 114.828427 92.828427) (end 112 94) (stroke (width 0.1) (type default)) (layer "Edge.Cuts"))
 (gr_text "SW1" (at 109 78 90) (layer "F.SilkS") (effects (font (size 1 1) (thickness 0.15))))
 (segment (start 102.4 84.4678) (end 102.2858 84.582) (width 0.25) (layer "F.Cu") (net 4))
 (segment (start 102.4 83) (end 102.4 84.4678) (width 0.25) (layer "F.Cu") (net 4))
 (via (at 102.2858 84.582) (size 0.8) (drill 0.4) (layers "F.Cu" "B.Cu") (free yes) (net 4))
 (segment (start 104 83) (end 106.379 83) (width 0.25) (layer "F.Cu") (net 3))
 (segment (start 108.7882 74.8284) (end 108.7882 81.0006) (width 0.25) (layer "F.Cu") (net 2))
 (segment (start 112 73.695) (end 109.9216 73.695) (width 0.25) (layer "F.Cu") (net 2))
 (segment (start 108.204 81.5848) (end 108.204 83) (width 0.25) (layer "F.Cu") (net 2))
 (segment (start 108.7882 81.0006) (end 108.204 81.5848) (width 0.25) (layer "F.Cu") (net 2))
 (segment (start 109.9216 73.695) (end 108.7882 74.8284) (width 0.25) (layer "F.Cu") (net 2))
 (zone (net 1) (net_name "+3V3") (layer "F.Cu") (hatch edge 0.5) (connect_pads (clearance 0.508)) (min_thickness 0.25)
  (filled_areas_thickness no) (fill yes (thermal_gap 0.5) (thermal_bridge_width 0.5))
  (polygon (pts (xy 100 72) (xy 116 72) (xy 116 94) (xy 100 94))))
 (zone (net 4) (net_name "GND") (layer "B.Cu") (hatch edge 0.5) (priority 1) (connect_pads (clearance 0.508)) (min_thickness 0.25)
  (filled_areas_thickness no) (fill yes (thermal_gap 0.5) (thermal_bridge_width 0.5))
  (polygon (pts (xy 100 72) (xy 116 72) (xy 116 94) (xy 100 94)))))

